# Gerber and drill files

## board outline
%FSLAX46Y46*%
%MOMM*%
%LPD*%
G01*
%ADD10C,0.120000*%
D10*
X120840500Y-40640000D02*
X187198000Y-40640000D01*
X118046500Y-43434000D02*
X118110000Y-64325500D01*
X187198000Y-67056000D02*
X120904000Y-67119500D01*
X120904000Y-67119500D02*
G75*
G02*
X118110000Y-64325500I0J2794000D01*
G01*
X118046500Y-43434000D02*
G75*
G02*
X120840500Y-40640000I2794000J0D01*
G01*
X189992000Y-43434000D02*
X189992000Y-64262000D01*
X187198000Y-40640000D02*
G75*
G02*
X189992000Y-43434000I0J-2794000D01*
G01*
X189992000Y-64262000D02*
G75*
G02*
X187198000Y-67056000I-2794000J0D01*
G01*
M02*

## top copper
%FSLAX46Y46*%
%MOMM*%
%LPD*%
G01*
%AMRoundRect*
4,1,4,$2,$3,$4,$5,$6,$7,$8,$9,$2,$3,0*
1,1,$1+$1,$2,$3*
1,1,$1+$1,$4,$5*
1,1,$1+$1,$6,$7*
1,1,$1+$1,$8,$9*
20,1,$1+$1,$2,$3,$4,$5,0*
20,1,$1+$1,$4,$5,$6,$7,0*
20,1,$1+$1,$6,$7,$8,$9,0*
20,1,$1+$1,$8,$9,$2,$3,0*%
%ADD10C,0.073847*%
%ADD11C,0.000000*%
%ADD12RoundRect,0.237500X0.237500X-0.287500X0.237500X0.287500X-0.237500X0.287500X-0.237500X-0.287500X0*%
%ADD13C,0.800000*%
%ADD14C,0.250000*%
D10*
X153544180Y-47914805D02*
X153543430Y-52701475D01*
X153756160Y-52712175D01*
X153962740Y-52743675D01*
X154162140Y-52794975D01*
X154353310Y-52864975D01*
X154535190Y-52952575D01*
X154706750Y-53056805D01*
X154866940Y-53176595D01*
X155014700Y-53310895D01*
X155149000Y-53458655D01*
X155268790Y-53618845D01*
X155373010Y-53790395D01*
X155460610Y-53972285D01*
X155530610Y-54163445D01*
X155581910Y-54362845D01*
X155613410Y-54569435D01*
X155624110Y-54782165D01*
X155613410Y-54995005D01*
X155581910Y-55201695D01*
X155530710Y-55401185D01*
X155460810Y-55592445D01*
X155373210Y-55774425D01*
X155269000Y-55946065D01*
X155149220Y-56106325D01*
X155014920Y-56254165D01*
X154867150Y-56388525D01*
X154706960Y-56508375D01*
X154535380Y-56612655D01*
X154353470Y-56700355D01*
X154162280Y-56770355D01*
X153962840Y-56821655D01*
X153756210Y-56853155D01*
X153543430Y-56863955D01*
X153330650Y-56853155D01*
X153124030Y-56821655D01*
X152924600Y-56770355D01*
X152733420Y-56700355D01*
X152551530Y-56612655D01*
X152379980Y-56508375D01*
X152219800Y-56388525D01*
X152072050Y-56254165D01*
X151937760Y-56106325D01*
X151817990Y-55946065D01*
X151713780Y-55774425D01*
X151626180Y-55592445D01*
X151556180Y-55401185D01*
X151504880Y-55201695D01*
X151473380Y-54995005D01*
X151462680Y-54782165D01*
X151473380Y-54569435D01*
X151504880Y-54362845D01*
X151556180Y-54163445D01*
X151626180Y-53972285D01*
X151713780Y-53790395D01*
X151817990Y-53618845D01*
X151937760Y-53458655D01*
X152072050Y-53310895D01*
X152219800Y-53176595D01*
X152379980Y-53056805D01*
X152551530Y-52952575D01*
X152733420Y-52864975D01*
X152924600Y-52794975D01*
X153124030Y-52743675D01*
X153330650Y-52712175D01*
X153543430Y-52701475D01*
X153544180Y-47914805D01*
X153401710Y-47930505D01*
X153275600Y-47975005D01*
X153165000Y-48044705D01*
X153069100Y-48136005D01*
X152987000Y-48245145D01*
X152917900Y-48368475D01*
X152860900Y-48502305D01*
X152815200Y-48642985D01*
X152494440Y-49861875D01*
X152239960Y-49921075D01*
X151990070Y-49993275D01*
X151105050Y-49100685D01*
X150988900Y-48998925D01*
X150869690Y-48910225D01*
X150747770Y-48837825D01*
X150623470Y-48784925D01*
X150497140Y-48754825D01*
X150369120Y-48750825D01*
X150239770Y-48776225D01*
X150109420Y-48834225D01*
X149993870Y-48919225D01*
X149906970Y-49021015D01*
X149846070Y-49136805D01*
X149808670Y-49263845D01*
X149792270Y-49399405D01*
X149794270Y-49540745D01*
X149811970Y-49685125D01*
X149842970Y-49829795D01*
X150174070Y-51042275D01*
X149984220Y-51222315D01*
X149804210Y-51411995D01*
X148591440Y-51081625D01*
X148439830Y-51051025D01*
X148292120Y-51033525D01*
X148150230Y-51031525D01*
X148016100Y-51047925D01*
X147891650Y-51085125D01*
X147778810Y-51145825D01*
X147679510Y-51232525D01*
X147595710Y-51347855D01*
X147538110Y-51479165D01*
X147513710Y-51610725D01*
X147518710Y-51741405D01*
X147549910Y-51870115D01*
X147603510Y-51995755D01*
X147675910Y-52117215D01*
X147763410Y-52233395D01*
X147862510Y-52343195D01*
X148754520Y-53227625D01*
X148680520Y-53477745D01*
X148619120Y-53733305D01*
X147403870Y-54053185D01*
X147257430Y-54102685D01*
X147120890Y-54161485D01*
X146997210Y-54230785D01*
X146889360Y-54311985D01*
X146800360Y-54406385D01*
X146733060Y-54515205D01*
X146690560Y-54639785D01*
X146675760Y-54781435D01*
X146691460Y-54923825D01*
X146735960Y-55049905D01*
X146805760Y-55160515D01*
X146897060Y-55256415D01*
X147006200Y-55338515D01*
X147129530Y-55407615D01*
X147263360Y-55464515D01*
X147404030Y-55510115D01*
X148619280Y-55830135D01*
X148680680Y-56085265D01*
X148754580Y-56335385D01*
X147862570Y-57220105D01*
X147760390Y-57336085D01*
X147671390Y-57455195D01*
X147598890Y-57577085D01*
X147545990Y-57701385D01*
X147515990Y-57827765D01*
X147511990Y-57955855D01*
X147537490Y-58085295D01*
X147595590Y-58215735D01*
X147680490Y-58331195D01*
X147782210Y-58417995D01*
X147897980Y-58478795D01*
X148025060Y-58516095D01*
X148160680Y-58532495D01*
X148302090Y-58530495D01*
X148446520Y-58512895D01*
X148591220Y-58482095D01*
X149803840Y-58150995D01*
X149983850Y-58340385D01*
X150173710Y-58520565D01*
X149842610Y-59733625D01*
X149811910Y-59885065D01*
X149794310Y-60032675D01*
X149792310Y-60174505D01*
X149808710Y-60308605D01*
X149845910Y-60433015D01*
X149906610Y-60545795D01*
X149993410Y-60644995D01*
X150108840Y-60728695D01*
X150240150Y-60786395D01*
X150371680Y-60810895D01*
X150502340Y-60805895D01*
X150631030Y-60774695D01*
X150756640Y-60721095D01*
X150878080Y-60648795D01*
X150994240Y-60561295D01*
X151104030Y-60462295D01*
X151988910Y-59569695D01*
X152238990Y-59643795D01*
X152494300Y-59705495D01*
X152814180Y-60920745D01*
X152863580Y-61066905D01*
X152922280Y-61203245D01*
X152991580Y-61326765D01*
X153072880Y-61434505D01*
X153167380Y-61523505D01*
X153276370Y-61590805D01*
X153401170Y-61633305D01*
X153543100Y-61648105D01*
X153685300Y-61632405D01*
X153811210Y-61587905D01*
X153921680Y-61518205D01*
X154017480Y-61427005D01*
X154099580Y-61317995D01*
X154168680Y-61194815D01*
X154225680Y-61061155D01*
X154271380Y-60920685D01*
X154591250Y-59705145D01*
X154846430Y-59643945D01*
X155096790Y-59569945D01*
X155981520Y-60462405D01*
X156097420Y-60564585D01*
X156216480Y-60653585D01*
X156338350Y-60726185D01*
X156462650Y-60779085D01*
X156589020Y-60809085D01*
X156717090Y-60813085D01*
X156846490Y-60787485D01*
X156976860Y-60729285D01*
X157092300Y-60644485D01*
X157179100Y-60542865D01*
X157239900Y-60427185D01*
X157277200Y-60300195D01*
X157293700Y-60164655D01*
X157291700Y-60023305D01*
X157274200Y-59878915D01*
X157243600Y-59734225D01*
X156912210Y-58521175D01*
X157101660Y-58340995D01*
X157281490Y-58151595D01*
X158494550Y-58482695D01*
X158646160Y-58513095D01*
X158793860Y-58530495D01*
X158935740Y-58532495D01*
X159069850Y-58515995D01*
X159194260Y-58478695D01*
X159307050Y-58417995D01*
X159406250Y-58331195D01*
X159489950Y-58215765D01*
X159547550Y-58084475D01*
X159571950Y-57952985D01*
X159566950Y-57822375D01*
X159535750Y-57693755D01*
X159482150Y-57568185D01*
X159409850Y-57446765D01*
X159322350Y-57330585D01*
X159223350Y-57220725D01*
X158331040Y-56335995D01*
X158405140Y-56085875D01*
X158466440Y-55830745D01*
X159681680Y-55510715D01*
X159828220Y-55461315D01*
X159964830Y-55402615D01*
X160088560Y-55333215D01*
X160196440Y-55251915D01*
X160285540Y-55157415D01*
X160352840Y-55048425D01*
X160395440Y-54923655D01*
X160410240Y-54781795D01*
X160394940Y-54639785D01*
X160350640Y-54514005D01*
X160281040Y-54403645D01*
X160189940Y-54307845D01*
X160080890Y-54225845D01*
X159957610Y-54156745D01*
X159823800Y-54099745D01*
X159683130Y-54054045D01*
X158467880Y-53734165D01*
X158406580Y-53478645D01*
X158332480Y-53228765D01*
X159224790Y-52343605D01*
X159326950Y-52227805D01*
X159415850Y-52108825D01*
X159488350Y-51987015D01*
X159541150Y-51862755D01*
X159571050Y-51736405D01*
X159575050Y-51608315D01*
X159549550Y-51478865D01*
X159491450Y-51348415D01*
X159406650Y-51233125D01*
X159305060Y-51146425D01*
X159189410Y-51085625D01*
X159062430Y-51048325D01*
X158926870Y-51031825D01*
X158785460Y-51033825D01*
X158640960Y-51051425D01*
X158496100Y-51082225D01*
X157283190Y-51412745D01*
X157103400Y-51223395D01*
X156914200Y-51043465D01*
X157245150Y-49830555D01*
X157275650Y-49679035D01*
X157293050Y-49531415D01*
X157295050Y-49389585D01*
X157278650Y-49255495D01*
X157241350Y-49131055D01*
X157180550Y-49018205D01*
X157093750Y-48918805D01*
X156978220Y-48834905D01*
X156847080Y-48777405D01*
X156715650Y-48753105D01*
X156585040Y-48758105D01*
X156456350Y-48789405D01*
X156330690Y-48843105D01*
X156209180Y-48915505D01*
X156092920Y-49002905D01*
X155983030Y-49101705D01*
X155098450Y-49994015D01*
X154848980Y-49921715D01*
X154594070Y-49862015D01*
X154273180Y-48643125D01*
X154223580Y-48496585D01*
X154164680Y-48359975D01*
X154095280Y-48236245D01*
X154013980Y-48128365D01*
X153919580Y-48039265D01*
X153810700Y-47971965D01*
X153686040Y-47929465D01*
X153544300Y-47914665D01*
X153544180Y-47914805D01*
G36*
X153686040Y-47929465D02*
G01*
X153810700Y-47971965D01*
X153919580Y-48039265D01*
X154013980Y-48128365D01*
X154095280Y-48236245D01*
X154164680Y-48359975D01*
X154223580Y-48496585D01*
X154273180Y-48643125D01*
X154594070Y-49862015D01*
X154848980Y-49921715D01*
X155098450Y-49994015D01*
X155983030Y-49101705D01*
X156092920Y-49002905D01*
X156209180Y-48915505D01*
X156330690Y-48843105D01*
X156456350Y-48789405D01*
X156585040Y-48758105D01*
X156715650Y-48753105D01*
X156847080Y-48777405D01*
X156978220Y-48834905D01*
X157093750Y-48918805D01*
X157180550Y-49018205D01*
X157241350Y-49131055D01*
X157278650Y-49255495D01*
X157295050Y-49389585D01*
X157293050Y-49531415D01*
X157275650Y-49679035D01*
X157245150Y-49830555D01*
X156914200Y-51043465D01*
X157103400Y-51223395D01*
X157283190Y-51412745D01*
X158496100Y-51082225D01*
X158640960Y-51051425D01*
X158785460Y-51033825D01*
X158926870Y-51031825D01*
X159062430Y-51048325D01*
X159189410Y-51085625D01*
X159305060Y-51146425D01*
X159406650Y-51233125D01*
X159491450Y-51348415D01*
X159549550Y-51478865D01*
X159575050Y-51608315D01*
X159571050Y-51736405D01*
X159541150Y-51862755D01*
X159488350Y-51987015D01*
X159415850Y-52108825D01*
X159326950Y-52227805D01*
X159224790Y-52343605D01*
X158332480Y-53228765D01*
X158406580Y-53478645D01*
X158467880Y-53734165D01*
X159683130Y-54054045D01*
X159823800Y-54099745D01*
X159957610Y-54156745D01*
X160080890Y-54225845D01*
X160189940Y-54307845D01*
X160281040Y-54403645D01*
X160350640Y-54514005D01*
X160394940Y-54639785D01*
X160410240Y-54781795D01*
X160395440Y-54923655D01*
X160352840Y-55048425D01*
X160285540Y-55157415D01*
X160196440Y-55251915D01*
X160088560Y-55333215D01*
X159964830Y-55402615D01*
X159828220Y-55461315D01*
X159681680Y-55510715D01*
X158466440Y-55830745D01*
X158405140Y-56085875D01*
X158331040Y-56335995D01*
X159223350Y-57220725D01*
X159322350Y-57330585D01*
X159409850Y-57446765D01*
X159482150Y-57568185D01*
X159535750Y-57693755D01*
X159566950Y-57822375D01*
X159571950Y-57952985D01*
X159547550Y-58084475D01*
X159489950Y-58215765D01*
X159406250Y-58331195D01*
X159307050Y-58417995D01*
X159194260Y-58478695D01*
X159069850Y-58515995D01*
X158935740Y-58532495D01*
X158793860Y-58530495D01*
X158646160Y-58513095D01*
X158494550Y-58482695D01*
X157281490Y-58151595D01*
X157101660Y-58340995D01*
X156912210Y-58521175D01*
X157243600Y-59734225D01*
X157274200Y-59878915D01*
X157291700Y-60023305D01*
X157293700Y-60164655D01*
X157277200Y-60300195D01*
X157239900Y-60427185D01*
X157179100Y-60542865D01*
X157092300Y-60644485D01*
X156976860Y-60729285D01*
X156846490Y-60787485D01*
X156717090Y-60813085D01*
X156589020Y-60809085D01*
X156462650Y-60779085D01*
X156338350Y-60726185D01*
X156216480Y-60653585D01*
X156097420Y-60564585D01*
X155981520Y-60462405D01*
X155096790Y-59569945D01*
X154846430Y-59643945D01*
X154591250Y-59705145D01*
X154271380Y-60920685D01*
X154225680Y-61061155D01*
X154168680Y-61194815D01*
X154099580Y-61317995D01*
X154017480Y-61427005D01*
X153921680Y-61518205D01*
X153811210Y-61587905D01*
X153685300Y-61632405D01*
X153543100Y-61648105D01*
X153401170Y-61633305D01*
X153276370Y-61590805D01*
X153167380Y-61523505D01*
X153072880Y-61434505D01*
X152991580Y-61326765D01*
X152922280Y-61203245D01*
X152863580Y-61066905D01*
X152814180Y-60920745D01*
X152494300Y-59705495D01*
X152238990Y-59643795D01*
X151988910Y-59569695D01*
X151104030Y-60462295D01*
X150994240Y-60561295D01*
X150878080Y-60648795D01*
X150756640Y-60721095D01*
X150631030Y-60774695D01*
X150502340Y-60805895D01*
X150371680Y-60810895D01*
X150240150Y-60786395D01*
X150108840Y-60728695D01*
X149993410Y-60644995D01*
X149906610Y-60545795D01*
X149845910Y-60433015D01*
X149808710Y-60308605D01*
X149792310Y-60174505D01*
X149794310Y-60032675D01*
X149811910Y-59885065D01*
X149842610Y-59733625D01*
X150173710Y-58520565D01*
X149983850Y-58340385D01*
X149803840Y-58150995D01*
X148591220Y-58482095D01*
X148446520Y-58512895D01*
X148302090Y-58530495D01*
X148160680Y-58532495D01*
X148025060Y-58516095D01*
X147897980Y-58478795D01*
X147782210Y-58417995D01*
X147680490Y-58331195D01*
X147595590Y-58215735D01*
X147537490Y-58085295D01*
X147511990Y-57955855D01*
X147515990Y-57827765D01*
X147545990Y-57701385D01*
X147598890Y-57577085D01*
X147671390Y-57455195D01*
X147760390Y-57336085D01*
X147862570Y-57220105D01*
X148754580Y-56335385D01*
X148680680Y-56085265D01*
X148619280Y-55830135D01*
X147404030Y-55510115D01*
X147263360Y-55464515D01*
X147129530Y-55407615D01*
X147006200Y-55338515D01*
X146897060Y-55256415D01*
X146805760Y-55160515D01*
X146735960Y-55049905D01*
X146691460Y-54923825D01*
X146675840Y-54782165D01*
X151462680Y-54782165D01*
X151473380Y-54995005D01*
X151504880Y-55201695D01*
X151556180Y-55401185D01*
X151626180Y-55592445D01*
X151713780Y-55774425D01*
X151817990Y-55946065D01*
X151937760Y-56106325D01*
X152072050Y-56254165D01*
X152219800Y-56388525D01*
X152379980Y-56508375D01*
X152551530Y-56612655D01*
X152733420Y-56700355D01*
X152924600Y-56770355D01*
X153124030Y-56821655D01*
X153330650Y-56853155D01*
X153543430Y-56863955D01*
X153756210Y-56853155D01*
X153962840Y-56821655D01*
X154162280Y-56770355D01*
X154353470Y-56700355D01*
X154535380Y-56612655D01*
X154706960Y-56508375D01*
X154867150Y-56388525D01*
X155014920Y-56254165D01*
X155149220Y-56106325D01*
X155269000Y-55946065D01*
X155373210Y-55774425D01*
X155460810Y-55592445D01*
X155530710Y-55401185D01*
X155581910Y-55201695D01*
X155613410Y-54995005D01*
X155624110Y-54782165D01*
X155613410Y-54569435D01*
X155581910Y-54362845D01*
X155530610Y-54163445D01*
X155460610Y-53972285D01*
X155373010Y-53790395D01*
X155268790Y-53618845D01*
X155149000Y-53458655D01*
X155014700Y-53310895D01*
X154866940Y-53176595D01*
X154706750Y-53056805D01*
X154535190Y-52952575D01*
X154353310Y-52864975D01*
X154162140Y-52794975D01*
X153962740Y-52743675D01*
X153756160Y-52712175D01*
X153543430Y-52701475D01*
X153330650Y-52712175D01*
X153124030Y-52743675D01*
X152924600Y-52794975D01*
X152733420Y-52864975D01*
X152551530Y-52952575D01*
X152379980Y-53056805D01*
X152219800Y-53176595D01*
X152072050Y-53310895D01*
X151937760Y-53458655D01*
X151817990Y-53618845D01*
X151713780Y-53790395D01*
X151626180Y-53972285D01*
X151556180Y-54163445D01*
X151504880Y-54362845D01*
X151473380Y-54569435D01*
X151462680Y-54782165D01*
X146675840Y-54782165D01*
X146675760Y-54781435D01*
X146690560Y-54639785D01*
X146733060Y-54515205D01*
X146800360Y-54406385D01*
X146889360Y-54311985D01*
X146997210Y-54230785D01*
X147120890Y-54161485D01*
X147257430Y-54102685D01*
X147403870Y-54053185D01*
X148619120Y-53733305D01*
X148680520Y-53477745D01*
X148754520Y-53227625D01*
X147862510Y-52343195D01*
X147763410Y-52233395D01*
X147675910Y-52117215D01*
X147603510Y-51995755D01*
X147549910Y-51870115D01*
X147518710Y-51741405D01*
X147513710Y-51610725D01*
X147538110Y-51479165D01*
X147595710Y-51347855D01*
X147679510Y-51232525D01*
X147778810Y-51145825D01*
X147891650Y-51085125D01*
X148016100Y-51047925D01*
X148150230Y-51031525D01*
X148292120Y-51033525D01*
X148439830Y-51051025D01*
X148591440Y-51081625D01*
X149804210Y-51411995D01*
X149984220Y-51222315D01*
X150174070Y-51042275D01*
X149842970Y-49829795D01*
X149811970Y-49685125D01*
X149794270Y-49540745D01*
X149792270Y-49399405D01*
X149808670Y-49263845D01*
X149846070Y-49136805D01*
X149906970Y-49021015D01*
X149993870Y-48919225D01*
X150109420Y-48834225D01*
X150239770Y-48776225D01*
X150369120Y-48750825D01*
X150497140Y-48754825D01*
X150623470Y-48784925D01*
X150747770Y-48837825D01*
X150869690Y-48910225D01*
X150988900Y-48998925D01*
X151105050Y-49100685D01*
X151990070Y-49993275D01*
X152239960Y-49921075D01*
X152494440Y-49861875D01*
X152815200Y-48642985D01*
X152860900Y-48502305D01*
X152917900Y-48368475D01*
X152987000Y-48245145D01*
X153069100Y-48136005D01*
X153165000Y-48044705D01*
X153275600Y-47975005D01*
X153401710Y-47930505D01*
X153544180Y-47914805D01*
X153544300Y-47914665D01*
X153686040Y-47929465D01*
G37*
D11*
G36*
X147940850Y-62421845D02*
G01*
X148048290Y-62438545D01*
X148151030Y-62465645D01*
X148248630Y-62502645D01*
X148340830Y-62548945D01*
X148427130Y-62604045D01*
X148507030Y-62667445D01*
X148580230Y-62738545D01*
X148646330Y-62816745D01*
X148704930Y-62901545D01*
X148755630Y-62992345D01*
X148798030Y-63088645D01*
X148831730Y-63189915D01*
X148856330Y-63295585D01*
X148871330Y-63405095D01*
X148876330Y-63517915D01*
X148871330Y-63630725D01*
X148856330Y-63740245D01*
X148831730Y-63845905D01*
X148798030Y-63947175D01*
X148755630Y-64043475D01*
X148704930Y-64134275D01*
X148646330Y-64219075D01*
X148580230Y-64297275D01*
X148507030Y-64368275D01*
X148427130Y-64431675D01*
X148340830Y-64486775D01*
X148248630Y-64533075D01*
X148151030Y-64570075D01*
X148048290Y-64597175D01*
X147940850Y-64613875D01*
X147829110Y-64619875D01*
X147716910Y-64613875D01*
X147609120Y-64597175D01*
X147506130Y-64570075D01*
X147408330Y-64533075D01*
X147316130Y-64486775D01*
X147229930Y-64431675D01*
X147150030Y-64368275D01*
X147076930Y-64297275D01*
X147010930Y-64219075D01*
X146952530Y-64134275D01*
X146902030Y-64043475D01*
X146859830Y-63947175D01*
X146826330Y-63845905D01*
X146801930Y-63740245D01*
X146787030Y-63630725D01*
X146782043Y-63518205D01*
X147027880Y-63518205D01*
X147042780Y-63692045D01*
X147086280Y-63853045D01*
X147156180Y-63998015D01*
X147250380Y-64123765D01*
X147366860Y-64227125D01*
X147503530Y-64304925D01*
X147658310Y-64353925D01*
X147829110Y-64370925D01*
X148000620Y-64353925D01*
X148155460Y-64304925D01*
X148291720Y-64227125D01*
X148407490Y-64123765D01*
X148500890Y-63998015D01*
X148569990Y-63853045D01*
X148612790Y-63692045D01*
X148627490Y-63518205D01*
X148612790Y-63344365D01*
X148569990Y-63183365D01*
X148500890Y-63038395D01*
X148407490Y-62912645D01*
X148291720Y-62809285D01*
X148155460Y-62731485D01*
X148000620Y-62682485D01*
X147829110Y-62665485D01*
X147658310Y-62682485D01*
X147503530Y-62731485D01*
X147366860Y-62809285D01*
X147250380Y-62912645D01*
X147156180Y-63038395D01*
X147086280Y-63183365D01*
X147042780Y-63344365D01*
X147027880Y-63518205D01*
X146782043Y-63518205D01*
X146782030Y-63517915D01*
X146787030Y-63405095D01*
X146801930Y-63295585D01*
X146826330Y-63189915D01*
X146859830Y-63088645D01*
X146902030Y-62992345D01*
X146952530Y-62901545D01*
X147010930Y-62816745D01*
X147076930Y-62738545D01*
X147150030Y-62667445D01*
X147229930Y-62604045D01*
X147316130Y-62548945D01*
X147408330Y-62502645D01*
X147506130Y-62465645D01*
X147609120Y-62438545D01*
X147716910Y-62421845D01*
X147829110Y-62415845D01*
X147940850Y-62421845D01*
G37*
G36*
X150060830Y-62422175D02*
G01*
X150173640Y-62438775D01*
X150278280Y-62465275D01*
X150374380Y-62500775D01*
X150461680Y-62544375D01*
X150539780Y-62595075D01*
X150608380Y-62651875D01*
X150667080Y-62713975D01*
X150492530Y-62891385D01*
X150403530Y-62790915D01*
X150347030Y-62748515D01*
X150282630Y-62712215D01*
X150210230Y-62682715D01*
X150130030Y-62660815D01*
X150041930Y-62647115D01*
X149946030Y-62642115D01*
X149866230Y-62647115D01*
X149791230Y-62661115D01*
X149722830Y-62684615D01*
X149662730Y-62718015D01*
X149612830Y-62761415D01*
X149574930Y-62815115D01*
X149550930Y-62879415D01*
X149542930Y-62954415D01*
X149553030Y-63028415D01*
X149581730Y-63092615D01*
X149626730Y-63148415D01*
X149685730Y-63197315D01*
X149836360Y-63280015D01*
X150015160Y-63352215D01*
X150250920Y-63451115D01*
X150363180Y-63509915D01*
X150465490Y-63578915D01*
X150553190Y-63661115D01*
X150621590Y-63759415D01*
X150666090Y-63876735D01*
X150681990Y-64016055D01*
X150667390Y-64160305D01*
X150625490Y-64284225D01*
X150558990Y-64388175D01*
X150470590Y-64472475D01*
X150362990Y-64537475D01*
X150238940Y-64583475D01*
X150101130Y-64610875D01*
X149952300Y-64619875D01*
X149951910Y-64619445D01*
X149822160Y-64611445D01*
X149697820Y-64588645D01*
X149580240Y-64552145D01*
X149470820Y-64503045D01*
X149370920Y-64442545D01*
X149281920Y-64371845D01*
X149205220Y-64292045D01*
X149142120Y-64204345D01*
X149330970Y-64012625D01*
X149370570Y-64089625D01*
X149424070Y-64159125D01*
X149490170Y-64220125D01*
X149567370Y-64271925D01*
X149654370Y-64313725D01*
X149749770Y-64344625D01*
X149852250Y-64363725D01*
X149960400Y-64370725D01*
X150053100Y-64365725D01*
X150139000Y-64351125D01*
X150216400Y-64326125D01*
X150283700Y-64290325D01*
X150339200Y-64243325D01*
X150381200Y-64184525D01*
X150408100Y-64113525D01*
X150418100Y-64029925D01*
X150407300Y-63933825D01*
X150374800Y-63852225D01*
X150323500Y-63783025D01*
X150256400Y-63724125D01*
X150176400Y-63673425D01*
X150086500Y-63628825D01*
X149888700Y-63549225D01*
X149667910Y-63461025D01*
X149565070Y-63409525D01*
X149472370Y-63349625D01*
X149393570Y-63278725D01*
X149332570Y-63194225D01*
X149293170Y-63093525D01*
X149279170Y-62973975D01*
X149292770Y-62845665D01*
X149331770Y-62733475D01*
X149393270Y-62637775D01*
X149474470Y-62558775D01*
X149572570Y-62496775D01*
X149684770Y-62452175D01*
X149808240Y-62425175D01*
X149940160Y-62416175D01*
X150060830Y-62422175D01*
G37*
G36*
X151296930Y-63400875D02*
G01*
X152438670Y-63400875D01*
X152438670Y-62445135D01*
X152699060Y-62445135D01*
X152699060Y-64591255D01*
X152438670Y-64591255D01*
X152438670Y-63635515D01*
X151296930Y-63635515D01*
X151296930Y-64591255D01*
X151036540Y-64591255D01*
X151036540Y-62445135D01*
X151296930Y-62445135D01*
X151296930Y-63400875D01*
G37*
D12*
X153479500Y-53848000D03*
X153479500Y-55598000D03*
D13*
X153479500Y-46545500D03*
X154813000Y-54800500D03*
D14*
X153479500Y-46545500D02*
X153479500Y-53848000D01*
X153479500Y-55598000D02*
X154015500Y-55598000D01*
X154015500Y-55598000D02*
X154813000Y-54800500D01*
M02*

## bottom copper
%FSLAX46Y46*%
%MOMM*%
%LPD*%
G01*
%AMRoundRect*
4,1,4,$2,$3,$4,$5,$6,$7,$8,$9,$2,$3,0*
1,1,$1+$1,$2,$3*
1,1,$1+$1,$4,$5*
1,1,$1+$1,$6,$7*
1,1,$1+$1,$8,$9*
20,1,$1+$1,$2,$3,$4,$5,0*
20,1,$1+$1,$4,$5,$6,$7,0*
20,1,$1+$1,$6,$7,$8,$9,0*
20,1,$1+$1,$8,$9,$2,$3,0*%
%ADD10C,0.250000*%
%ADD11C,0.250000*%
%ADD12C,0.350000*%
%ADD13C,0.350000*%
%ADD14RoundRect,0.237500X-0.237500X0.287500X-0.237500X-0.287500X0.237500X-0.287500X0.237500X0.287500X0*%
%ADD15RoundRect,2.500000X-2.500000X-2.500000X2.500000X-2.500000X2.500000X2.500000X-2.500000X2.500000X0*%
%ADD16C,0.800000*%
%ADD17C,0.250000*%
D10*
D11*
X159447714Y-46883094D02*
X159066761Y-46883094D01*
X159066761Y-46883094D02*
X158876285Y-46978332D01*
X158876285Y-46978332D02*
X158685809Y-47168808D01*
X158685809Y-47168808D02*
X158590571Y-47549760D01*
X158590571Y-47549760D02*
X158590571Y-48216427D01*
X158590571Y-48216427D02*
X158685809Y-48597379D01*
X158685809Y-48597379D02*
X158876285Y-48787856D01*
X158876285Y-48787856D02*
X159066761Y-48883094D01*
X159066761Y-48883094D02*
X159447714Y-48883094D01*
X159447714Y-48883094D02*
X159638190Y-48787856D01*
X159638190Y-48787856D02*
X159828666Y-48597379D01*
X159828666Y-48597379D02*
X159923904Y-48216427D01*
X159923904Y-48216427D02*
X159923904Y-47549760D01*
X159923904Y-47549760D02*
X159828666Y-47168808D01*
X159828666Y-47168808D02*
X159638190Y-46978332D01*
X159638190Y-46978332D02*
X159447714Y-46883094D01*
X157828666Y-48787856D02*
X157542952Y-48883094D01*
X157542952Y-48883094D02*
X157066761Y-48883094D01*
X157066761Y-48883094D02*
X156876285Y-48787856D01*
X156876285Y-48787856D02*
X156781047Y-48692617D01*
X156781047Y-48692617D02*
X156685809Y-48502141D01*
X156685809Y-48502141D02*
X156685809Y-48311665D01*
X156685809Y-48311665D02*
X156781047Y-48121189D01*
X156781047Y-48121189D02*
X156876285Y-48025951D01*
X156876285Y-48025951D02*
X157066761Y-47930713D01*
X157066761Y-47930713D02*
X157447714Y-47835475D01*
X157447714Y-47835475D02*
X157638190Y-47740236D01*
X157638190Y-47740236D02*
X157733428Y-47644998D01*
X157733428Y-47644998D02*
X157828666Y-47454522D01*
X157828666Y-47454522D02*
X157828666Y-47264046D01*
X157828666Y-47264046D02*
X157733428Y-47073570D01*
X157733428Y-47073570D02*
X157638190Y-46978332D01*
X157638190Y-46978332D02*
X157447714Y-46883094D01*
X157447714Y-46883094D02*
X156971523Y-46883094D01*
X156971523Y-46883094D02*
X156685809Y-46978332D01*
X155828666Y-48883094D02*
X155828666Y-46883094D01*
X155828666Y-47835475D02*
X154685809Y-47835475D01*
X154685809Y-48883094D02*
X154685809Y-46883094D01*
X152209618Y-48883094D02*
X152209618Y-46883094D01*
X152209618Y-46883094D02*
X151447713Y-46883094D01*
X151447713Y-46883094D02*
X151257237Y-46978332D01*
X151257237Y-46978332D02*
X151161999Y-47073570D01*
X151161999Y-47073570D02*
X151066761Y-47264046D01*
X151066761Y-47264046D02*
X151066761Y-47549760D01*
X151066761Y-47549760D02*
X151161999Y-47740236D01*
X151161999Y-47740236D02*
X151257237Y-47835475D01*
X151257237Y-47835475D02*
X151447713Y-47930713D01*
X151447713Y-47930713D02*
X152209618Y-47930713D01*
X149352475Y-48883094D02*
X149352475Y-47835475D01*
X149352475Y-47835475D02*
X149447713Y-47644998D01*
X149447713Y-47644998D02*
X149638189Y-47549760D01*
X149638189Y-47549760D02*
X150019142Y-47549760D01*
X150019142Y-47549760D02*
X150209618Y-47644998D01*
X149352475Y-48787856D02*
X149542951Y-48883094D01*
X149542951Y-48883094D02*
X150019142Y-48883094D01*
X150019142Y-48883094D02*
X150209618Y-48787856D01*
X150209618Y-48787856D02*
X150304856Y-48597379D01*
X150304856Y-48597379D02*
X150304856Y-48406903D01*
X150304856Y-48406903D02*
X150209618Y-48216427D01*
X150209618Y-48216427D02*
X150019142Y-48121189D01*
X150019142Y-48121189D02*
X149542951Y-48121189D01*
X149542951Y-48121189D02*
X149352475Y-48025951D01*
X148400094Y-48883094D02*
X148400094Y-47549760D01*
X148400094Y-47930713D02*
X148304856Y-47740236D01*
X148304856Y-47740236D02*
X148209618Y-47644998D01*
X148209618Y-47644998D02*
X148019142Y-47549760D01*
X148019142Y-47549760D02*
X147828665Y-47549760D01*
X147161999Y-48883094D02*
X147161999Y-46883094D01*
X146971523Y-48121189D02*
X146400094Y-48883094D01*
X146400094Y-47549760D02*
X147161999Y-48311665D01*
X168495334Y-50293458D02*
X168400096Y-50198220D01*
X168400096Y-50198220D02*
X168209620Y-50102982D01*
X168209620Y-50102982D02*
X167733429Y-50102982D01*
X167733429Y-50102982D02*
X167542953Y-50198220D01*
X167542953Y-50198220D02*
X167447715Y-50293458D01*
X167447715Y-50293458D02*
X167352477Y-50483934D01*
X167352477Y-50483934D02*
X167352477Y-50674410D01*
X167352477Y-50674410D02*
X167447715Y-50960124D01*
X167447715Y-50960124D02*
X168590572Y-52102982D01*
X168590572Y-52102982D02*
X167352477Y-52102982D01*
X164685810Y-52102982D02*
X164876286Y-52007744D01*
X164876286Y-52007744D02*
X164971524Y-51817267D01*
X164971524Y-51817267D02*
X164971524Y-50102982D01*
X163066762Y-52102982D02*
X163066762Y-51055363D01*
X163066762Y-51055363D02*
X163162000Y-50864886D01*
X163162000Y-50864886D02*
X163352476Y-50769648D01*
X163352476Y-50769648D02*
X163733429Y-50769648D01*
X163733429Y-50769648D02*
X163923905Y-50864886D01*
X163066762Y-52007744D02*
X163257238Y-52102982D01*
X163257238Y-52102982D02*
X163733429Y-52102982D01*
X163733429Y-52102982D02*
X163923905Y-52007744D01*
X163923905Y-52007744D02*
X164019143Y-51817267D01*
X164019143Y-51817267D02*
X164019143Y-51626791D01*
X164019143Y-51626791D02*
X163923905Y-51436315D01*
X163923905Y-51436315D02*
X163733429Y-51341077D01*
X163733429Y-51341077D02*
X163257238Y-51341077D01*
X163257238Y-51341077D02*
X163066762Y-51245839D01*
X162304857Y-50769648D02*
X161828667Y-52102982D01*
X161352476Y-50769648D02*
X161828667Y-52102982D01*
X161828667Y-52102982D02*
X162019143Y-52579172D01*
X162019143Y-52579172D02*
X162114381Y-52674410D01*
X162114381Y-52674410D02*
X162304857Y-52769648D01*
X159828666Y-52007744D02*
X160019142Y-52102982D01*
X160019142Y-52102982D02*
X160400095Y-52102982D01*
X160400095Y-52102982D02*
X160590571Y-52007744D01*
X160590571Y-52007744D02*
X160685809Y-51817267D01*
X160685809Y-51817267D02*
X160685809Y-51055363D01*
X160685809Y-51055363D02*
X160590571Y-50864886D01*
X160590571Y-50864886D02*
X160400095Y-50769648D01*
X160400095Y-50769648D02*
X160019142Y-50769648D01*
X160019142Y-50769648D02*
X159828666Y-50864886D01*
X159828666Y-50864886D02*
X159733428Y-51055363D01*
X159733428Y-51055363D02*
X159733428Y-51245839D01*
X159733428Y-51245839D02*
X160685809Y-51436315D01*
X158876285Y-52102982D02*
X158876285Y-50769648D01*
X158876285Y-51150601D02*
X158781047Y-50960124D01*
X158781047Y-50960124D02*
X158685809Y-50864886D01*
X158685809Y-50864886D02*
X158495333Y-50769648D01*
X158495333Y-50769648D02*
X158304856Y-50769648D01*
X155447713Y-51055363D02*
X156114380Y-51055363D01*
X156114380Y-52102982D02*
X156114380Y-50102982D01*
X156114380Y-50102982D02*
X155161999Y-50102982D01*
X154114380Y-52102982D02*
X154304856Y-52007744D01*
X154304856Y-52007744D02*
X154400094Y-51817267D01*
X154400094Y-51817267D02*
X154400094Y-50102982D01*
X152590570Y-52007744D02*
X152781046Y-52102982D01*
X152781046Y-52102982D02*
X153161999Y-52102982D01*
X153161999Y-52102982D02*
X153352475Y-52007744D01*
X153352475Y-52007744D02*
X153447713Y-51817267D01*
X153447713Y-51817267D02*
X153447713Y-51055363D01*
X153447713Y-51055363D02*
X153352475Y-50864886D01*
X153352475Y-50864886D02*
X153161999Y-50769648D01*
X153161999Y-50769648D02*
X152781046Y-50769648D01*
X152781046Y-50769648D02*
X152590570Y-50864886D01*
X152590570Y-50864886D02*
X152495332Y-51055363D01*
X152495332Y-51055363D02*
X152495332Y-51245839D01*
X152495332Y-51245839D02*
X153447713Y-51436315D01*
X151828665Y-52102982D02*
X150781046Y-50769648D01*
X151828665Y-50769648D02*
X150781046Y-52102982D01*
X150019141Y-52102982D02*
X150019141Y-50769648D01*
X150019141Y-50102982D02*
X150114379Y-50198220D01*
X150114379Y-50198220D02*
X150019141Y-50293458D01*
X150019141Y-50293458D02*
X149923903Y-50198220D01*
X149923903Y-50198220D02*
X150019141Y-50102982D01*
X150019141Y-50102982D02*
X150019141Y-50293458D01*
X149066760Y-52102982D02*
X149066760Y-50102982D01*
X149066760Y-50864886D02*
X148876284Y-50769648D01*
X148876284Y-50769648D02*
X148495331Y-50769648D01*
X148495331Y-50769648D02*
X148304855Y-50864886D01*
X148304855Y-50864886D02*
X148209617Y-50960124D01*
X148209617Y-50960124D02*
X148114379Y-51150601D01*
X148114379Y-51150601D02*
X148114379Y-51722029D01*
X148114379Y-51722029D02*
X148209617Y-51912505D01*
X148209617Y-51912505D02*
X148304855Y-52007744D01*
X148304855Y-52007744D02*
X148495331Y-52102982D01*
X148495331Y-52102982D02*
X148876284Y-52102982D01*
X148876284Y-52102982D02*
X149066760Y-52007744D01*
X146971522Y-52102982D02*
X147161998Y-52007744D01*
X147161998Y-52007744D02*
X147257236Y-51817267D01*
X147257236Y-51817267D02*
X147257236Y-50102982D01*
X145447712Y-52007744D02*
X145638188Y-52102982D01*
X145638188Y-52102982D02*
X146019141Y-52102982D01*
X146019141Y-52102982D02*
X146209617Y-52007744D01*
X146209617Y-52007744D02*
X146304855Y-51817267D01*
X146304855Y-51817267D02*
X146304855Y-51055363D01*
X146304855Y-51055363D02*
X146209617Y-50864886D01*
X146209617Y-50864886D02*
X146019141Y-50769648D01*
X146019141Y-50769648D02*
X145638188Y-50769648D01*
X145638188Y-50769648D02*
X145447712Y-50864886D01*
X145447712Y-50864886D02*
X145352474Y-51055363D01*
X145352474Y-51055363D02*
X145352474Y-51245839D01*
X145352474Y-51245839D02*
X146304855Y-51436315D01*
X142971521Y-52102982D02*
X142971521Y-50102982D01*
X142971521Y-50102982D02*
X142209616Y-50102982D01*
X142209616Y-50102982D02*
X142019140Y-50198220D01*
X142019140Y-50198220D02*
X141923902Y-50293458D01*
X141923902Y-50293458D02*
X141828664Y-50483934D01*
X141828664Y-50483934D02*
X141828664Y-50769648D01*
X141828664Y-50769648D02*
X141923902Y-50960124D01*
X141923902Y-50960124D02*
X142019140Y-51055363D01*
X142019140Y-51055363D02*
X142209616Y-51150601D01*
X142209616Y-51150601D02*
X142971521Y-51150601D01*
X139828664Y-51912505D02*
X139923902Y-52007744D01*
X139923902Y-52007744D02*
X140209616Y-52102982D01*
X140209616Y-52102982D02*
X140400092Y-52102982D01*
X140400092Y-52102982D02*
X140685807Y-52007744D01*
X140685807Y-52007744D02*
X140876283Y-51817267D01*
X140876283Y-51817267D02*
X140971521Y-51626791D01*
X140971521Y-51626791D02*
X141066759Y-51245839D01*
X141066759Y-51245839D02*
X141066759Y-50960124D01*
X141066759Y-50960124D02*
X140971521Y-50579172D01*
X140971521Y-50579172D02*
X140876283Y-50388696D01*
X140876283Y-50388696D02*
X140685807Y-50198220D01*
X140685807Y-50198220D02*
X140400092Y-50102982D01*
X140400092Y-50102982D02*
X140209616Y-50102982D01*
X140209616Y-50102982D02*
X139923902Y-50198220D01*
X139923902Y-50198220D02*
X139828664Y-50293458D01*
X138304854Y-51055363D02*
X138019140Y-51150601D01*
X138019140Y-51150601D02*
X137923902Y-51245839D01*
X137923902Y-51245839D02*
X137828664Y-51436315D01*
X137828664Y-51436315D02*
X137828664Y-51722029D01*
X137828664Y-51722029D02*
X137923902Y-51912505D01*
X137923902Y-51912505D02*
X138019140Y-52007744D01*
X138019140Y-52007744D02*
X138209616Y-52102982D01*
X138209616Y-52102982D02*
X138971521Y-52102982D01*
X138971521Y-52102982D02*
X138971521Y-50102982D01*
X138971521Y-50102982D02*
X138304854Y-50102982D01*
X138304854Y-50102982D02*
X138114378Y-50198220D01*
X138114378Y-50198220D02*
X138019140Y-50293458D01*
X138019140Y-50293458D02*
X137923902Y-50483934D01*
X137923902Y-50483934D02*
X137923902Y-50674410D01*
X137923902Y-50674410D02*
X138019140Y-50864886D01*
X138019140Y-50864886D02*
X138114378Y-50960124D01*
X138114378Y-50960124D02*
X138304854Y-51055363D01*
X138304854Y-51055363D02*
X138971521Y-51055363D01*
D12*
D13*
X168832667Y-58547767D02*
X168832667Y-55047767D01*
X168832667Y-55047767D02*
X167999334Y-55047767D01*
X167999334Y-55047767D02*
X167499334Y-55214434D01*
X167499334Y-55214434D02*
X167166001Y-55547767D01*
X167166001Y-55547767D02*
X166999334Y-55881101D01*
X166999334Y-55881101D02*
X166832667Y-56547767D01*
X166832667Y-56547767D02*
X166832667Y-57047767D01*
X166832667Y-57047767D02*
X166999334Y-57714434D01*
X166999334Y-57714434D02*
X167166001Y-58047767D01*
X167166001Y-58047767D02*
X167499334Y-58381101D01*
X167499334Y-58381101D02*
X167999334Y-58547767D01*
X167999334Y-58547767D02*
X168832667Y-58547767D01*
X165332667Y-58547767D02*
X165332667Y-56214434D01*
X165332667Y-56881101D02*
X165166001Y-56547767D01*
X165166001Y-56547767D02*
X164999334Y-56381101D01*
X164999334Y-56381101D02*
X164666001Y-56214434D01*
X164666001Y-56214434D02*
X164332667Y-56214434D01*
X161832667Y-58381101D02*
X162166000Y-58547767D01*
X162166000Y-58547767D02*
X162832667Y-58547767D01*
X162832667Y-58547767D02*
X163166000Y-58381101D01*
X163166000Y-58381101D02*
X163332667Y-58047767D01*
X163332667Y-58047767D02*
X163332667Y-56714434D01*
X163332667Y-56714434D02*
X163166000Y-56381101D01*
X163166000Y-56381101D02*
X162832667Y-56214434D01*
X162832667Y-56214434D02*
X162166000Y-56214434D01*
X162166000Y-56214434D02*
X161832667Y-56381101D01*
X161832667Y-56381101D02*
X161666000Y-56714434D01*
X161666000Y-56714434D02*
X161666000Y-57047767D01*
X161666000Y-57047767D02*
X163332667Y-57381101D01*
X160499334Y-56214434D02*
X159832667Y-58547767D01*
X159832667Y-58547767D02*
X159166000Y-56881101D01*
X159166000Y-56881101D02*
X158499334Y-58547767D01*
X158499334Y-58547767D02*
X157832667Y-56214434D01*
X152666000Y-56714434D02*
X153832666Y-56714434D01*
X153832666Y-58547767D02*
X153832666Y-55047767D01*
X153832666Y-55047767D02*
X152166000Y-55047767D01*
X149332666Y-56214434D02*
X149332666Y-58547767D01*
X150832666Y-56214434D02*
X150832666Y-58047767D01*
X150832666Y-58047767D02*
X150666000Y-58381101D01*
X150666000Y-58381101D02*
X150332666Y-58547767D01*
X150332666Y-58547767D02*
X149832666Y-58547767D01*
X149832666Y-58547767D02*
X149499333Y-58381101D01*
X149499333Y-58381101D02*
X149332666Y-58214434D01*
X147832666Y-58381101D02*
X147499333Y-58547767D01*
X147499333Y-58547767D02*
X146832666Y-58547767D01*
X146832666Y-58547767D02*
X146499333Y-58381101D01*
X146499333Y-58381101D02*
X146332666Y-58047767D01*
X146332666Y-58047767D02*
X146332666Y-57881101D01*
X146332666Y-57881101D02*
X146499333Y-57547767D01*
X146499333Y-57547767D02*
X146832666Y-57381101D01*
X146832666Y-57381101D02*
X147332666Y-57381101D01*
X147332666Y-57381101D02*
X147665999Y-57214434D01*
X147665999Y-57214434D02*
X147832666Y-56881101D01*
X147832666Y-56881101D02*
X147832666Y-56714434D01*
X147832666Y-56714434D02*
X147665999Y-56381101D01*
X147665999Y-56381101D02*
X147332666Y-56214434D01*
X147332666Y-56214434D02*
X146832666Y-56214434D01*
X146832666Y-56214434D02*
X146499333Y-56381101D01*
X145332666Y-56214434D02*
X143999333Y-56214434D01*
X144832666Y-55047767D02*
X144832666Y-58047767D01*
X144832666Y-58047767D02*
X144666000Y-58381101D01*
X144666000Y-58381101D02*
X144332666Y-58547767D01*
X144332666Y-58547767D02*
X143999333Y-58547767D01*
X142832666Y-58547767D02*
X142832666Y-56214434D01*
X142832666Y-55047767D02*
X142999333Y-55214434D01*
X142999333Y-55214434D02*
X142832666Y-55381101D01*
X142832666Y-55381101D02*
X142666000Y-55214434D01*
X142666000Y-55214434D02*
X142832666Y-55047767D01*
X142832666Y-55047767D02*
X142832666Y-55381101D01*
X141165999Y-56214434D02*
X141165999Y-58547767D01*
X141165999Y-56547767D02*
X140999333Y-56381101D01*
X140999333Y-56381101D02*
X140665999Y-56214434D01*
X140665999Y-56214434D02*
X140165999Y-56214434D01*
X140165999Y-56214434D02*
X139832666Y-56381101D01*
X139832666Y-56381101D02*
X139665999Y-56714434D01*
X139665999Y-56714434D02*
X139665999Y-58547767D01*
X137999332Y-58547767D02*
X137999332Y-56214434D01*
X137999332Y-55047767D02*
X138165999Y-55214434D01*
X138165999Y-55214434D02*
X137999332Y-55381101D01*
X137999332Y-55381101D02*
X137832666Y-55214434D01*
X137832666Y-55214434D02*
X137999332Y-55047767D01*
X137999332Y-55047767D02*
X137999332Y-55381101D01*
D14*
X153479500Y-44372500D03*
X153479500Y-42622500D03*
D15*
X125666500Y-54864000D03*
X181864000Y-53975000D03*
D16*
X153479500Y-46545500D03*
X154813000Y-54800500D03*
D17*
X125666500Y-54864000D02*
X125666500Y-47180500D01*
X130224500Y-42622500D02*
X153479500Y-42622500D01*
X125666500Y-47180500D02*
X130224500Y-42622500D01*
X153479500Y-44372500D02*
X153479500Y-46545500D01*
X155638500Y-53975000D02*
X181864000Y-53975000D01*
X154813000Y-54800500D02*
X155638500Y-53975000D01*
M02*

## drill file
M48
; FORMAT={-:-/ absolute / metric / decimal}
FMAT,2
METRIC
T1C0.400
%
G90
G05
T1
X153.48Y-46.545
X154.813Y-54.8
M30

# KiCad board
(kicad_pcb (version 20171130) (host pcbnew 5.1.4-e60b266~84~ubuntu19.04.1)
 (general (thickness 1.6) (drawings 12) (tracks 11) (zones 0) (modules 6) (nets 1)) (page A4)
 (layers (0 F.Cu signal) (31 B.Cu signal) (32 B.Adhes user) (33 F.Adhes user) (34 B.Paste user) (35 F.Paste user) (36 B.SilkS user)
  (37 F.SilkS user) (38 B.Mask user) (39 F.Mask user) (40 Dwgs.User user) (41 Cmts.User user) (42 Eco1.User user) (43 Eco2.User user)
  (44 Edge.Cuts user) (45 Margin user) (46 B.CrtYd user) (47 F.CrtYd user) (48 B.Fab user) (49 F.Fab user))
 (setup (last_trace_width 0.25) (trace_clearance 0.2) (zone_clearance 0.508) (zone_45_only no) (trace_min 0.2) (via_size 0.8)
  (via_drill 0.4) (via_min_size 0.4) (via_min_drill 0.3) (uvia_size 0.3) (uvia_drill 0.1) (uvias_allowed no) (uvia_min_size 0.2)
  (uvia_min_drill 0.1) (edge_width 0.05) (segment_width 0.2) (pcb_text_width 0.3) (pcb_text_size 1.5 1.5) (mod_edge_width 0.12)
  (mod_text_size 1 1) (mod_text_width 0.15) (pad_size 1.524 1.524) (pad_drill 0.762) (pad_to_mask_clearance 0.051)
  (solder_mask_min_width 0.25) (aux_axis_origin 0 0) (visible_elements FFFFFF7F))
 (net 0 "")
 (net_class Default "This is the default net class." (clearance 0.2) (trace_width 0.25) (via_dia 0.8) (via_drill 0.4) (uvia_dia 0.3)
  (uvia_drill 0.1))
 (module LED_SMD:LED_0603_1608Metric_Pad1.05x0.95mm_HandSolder (layer F.Cu) (at 153.4795 54.723 90)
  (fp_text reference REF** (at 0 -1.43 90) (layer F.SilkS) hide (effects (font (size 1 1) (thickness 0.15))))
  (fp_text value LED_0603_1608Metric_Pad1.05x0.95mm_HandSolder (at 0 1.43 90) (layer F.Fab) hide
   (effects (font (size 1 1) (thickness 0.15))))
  (pad 2 smd roundrect (at 0.875 0 90) (size 1.05 0.95) (layers F.Cu F.Paste F.Mask) (roundrect_rratio 0.25))
  (pad 1 smd roundrect (at -0.875 0 90) (size 1.05 0.95) (layers F.Cu F.Paste F.Mask) (roundrect_rratio 0.25)))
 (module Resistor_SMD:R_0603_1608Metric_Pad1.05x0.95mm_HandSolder (layer B.Cu) (at 153.4795 43.4975 270)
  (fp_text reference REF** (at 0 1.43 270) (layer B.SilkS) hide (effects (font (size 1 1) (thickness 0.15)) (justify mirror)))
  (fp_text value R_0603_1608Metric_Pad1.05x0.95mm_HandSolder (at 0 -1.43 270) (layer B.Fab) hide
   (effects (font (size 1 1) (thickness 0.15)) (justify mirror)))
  (pad 2 smd roundrect (at 0.875 0 270) (size 1.05 0.95) (layers B.Cu B.Paste B.Mask) (roundrect_rratio 0.25))
  (pad 1 smd roundrect (at -0.875 0 270) (size 1.05 0.95) (layers B.Cu B.Paste B.Mask) (roundrect_rratio 0.25)))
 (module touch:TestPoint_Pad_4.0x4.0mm (layer B.Cu) (at 125.6665 54.864)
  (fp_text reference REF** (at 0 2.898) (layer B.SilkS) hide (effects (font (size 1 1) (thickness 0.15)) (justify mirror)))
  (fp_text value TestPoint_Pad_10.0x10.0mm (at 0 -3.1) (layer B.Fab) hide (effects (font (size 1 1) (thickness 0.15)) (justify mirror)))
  (pad 1 smd roundrect (at 0 0) (size 10 10) (layers B.Cu B.Mask) (roundrect_rratio 0.25)))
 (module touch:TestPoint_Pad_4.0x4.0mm (layer B.Cu) (at 181.864 53.975)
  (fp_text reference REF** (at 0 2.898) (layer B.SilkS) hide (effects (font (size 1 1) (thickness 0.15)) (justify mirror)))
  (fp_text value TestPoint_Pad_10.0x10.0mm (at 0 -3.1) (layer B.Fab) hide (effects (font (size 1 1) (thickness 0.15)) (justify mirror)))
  (pad 1 smd roundrect (at 0 0) (size 10 10) (layers B.Cu B.Mask) (roundrect_rratio 0.25)))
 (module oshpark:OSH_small (layer F.Cu) (at 153.543 56.3245)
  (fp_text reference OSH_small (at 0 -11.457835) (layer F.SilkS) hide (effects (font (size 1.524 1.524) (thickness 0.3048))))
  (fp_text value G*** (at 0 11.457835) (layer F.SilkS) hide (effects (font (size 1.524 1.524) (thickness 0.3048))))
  (fp_poly
   (pts (xy 0.00118 -8.409695) (xy 0.00043 -3.623025) (xy 0.21316 -3.612325) (xy 0.41974 -3.580825) (xy 0.61914 -3.529525)
    (xy 0.81031 -3.459525) (xy 0.99219 -3.371925) (xy 1.16375 -3.267695) (xy 1.32394 -3.147905) (xy 1.4717 -3.013605) (xy 1.606 -2.865845)
    (xy 1.72579 -2.705655) (xy 1.83001 -2.534105) (xy 1.91761 -2.352215) (xy 1.98761 -2.161055) (xy 2.03891 -1.961655)
    (xy 2.07041 -1.755065) (xy 2.08111 -1.542335) (xy 2.07041 -1.329495) (xy 2.03891 -1.122805) (xy 1.98771 -0.923315)
    (xy 1.91781 -0.732055) (xy 1.83021 -0.550075) (xy 1.726 -0.378435) (xy 1.60622 -0.218175) (xy 1.47192 -0.070335) (xy 1.32415 0.064025)
    (xy 1.16396 0.183875) (xy 0.99238 0.288155) (xy 0.81047 0.375855) (xy 0.61928 0.445855) (xy 0.41984 0.497155) (xy 0.21321 0.528655)
    (xy 0.00043 0.539455) (xy -0.21235 0.528655) (xy -0.41897 0.497155) (xy -0.6184 0.445855) (xy -0.80958 0.375855) (xy -0.99147 0.288155)
    (xy -1.16302 0.183875) (xy -1.3232 0.064025) (xy -1.47095 -0.070335) (xy -1.60524 -0.218175) (xy -1.72501 -0.378435)
    (xy -1.82922 -0.550075) (xy -1.91682 -0.732055) (xy -1.98682 -0.923315) (xy -2.03812 -1.122805) (xy -2.06962 -1.329495)
    (xy -2.08032 -1.542335) (xy -2.06962 -1.755065) (xy -2.03812 -1.961655) (xy -1.98682 -2.161055) (xy -1.91682 -2.352215)
    (xy -1.82922 -2.534105) (xy -1.72501 -2.705655) (xy -1.60524 -2.865845) (xy -1.47095 -3.013605) (xy -1.3232 -3.147905)
    (xy -1.16302 -3.267695) (xy -0.99147 -3.371925) (xy -0.80958 -3.459525) (xy -0.6184 -3.529525) (xy -0.41897 -3.580825)
    (xy -0.21235 -3.612325) (xy 0.00043 -3.623025) (xy 0.00118 -8.409695) (xy -0.14129 -8.393995) (xy -0.2674 -8.349495)
    (xy -0.378 -8.279795) (xy -0.4739 -8.188495) (xy -0.556 -8.079355) (xy -0.6251 -7.956025) (xy -0.6821 -7.822195) (xy -0.7278 -7.681515)
    (xy -1.04856 -6.462625) (xy -1.30304 -6.403425) (xy -1.55293 -6.331225) (xy -2.43795 -7.223815) (xy -2.5541 -7.325575)
    (xy -2.67331 -7.414275) (xy -2.79523 -7.486675) (xy -2.91953 -7.539575) (xy -3.04586 -7.569675) (xy -3.17388 -7.573675)
    (xy -3.30323 -7.548275) (xy -3.43358 -7.490275) (xy -3.54913 -7.405275) (xy -3.63603 -7.303485) (xy -3.69693 -7.187695)
    (xy -3.73433 -7.060655) (xy -3.75073 -6.925095) (xy -3.74873 -6.783755) (xy -3.73103 -6.639375) (xy -3.70003 -6.494705)
    (xy -3.36893 -5.282225) (xy -3.55878 -5.102185) (xy -3.73879 -4.912505) (xy -4.95156 -5.242875) (xy -5.10317 -5.273475)
    (xy -5.25088 -5.290975) (xy -5.39277 -5.292975) (xy -5.5269 -5.276575) (xy -5.65135 -5.239375) (xy -5.76419 -5.178675)
    (xy -5.86349 -5.091975) (xy -5.94729 -4.976645) (xy -6.00489 -4.845335) (xy -6.02929 -4.713775) (xy -6.02429 -4.583095)
    (xy -5.99309 -4.454385) (xy -5.93949 -4.328745) (xy -5.86709 -4.207285) (xy -5.77959 -4.091105) (xy -5.68049 -3.981305)
    (xy -4.78848 -3.096875) (xy -4.86248 -2.846755) (xy -4.92388 -2.591195) (xy -6.13913 -2.271315) (xy -6.28557 -2.221815)
    (xy -6.42211 -2.163015) (xy -6.54579 -2.093715) (xy -6.65364 -2.012515) (xy -6.74264 -1.918115) (xy -6.80994 -1.809295)
    (xy -6.85244 -1.684715) (xy -6.86724 -1.543065) (xy -6.85154 -1.400675) (xy -6.80704 -1.274595) (xy -6.73724 -1.163985)
    (xy -6.64594 -1.068085) (xy -6.5368 -0.985985) (xy -6.41347 -0.916885) (xy -6.27964 -0.859985) (xy -6.13897 -0.814385)
    (xy -4.92372 -0.494365) (xy -4.86232 -0.239235) (xy -4.78842 0.010885) (xy -5.68043 0.895605) (xy -5.78261 1.011585)
    (xy -5.87161 1.130695) (xy -5.94411 1.252585) (xy -5.99701 1.376885) (xy -6.02701 1.503265) (xy -6.03101 1.631355)
    (xy -6.00551 1.760795) (xy -5.94741 1.891235) (xy -5.86251 2.006695) (xy -5.76079 2.093495) (xy -5.64502 2.154295)
    (xy -5.51794 2.191595) (xy -5.38232 2.207995) (xy -5.24091 2.205995) (xy -5.09648 2.188395) (xy -4.95178 2.157595)
    (xy -3.73916 1.826495) (xy -3.55915 2.015885) (xy -3.36929 2.196065) (xy -3.70039 3.409125) (xy -3.73109 3.560565)
    (xy -3.74869 3.708175) (xy -3.75069 3.850005) (xy -3.73429 3.984105) (xy -3.69709 4.108515) (xy -3.63639 4.221295)
    (xy -3.54959 4.320495) (xy -3.43416 4.404195) (xy -3.30285 4.461895) (xy -3.17132 4.486395) (xy -3.04066 4.481395)
    (xy -2.91197 4.450195) (xy -2.78636 4.396595) (xy -2.66492 4.324295) (xy -2.54876 4.236795) (xy -2.43897 4.137795)
    (xy -1.55409 3.245195) (xy -1.30401 3.319295) (xy -1.0487 3.380995) (xy -0.72882 4.596245) (xy -0.67942 4.742405) (xy -0.62072 4.878745)
    (xy -0.55142 5.002265) (xy -0.47012 5.110005) (xy -0.37562 5.199005) (xy -0.26663 5.266305) (xy -0.14183 5.308805) (xy 0.0001 5.323605)
    (xy 0.1423 5.307905) (xy 0.26821 5.263405) (xy 0.37868 5.193705) (xy 0.47448 5.102505) (xy 0.55658 4.993495) (xy 0.62568 4.870315)
    (xy 0.68268 4.736655) (xy 0.72838 4.596185) (xy 1.04825 3.380645) (xy 1.30343 3.319445) (xy 1.55379 3.245445) (xy 2.43852 4.137905)
    (xy 2.55442 4.240085) (xy 2.67348 4.329085) (xy 2.79535 4.401685) (xy 2.91965 4.454585) (xy 3.04602 4.484585) (xy 3.17409 4.488585)
    (xy 3.30349 4.462985) (xy 3.43386 4.404785) (xy 3.5493 4.319985) (xy 3.6361 4.218365) (xy 3.6969 4.102685) (xy 3.7342 3.975695)
    (xy 3.7507 3.840155) (xy 3.7487 3.698805) (xy 3.7312 3.554415) (xy 3.7006 3.409725) (xy 3.36921 2.196675) (xy 3.55866 2.016495)
    (xy 3.73849 1.827095) (xy 4.95155 2.158195) (xy 5.10316 2.188595) (xy 5.25086 2.205995) (xy 5.39274 2.207995) (xy 5.52685 2.191495)
    (xy 5.65126 2.154195) (xy 5.76405 2.093495) (xy 5.86325 2.006695) (xy 5.94695 1.891265) (xy 6.00455 1.759975) (xy 6.02895 1.628485)
    (xy 6.02395 1.497875) (xy 5.99275 1.369255) (xy 5.93915 1.243685) (xy 5.86685 1.122265) (xy 5.77935 1.006085) (xy 5.68035 0.896225)
    (xy 4.78804 0.011495) (xy 4.86214 -0.238625) (xy 4.92344 -0.493755) (xy 6.13868 -0.813785) (xy 6.28522 -0.863185) (xy 6.42183 -0.921885)
    (xy 6.54556 -0.991285) (xy 6.65344 -1.072585) (xy 6.74254 -1.167085) (xy 6.80984 -1.276075) (xy 6.85244 -1.400845)
    (xy 6.86724 -1.542705) (xy 6.85194 -1.684715) (xy 6.80764 -1.810495) (xy 6.73804 -1.920855) (xy 6.64694 -2.016655)
    (xy 6.53789 -2.098655) (xy 6.41461 -2.167755) (xy 6.2808 -2.224755) (xy 6.14013 -2.270455) (xy 4.92488 -2.590335) (xy 4.86358 -2.845855)
    (xy 4.78948 -3.095735) (xy 5.68179 -3.980895) (xy 5.78395 -4.096695) (xy 5.87285 -4.215675) (xy 5.94535 -4.337485)
    (xy 5.99815 -4.461745) (xy 6.02805 -4.588095) (xy 6.03205 -4.716185) (xy 6.00655 -4.845635) (xy 5.94845 -4.976085)
    (xy 5.86365 -5.091375) (xy 5.76206 -5.178075) (xy 5.64641 -5.238875) (xy 5.51943 -5.276175) (xy 5.38387 -5.292675)
    (xy 5.24246 -5.290675) (xy 5.09796 -5.273075) (xy 4.9531 -5.242275) (xy 3.74019 -4.911755) (xy 3.5604 -5.101105) (xy 3.3712 -5.281035)
    (xy 3.70215 -6.493945) (xy 3.73265 -6.645465) (xy 3.75005 -6.793085) (xy 3.75205 -6.934915) (xy 3.73565 -7.069005)
    (xy 3.69835 -7.193445) (xy 3.63755 -7.306295) (xy 3.55075 -7.405695) (xy 3.43522 -7.489595) (xy 3.30408 -7.547095)
    (xy 3.17265 -7.571395) (xy 3.04204 -7.566395) (xy 2.91335 -7.535095) (xy 2.78769 -7.481395) (xy 2.66618 -7.408995)
    (xy 2.54992 -7.321595) (xy 2.44003 -7.222795) (xy 1.55545 -6.330485) (xy 1.30598 -6.402785) (xy 1.05107 -6.462485)
    (xy 0.73018 -7.681375) (xy 0.68058 -7.827915) (xy 0.62168 -7.964525) (xy 0.55228 -8.088255) (xy 0.47098 -8.196135)
    (xy 0.37658 -8.285235) (xy 0.2677 -8.352535) (xy 0.14304 -8.395035) (xy 0.0013 -8.409835) (xy 0.00118 -8.409695))
   (layer F.Cu) (width 0.073847))
  (fp_poly
   (pts (xy -5.71389 8.295375) (xy -5.71389 8.046425) (xy -5.88469 8.029425) (xy -6.03947 7.980425) (xy -6.17614 7.902625)
    (xy -6.29262 7.799265) (xy -6.38682 7.673515) (xy -6.45672 7.528545) (xy -6.50022 7.367545) (xy -6.51512 7.193705)
    (xy -6.50022 7.019865) (xy -6.45672 6.858865) (xy -6.38682 6.713895) (xy -6.29262 6.588145) (xy -6.17614 6.484785)
    (xy -6.03947 6.406985) (xy -5.88469 6.357985) (xy -5.71389 6.340985) (xy -5.54238 6.357985) (xy -5.38754 6.406985)
    (xy -5.25128 6.484785) (xy -5.13551 6.588145) (xy -5.04211 6.713895) (xy -4.97301 6.858865) (xy -4.93021 7.019865)
    (xy -4.91551 7.193705) (xy -4.93021 7.367545) (xy -4.97301 7.528545) (xy -5.04211 7.673515) (xy -5.13551 7.799265)
    (xy -5.25128 7.902625) (xy -5.38754 7.980425) (xy -5.54238 8.029425) (xy -5.71389 8.046425) (xy -5.71389 8.295375)
    (xy -5.60215 8.289375) (xy -5.49471 8.272675) (xy -5.39197 8.245575) (xy -5.29437 8.208575) (xy -5.20217 8.162275)
    (xy -5.11587 8.107175) (xy -5.03597 8.043775) (xy -4.96277 7.972775) (xy -4.89667 7.894575) (xy -4.83807 7.809775)
    (xy -4.78737 7.718975) (xy -4.74497 7.622675) (xy -4.71127 7.521405) (xy -4.68667 7.415745) (xy -4.67167 7.306225)
    (xy -4.66667 7.193415) (xy -4.67167 7.080595) (xy -4.68667 6.971085) (xy -4.71127 6.865415) (xy -4.74497 6.764145)
    (xy -4.78737 6.667845) (xy -4.83807 6.577045) (xy -4.89667 6.492245) (xy -4.96277 6.414045) (xy -5.03597 6.342945)
    (xy -5.11587 6.279545) (xy -5.20217 6.224445) (xy -5.29437 6.178145) (xy -5.39197 6.141145) (xy -5.49471 6.114045)
    (xy -5.60215 6.097345) (xy -5.71389 6.091345) (xy -5.82609 6.097345) (xy -5.93388 6.114045) (xy -6.03687 6.141145)
    (xy -6.13467 6.178145) (xy -6.22687 6.224445) (xy -6.31307 6.279545) (xy -6.39297 6.342945) (xy -6.46607 6.414045)
    (xy -6.53207 6.492245) (xy -6.59047 6.577045) (xy -6.64097 6.667845) (xy -6.68317 6.764145) (xy -6.71667 6.865415)
    (xy -6.74107 6.971085) (xy -6.75597 7.080595) (xy -6.76097 7.193415) (xy -6.75597 7.306225) (xy -6.74107 7.415745)
    (xy -6.71667 7.521405) (xy -6.68317 7.622675) (xy -6.64097 7.718975) (xy -6.59047 7.809775) (xy -6.53207 7.894575)
    (xy -6.46607 7.972775) (xy -6.39297 8.043775) (xy -6.31307 8.107175) (xy -6.22687 8.162275) (xy -6.13467 8.208575)
    (xy -6.03687 8.245575) (xy -5.93388 8.272675) (xy -5.82609 8.289375) (xy -5.71389 8.295375))
   (layer F.Cu) (width 0))
  (fp_poly
   (pts (xy -3.5907 8.295375) (xy -3.44187 8.286375) (xy -3.30406 8.258975) (xy -3.18001 8.212975) (xy -3.07241 8.147975)
    (xy -2.98401 8.063675) (xy -2.91751 7.959725) (xy -2.87561 7.835805) (xy -2.86101 7.691555) (xy -2.87691 7.552235)
    (xy -2.92141 7.434915) (xy -2.98981 7.336615) (xy -3.07751 7.254415) (xy -3.17982 7.185415) (xy -3.29208 7.126615)
    (xy -3.52784 7.027715) (xy -3.70664 6.955515) (xy -3.85727 6.872815) (xy -3.91627 6.823915) (xy -3.96127 6.768115)
    (xy -3.98997 6.703915) (xy -4.00007 6.629915) (xy -3.99207 6.554915) (xy -3.96807 6.490615) (xy -3.93017 6.436915)
    (xy -3.88027 6.393515) (xy -3.82017 6.360115) (xy -3.75177 6.336615) (xy -3.67677 6.322615) (xy -3.59697 6.317615)
    (xy -3.50107 6.322615) (xy -3.41297 6.336315) (xy -3.33277 6.358215) (xy -3.26037 6.387715) (xy -3.19597 6.424015)
    (xy -3.13947 6.466415) (xy -3.05047 6.566885) (xy -2.87592 6.389475) (xy -2.93462 6.327375) (xy -3.00322 6.270575)
    (xy -3.08132 6.219875) (xy -3.16862 6.176275) (xy -3.26472 6.140775) (xy -3.36936 6.114275) (xy -3.48217 6.097675)
    (xy -3.60284 6.091675) (xy -3.73476 6.100675) (xy -3.85823 6.127675) (xy -3.97043 6.172275) (xy -4.06853 6.234275)
    (xy -4.14973 6.313275) (xy -4.21123 6.408975) (xy -4.25023 6.521165) (xy -4.26383 6.649475) (xy -4.24983 6.769025)
    (xy -4.21043 6.869725) (xy -4.14943 6.954225) (xy -4.07063 7.025125) (xy -3.97793 7.085025) (xy -3.87509 7.136525) (xy -3.6543 7.224725)
    (xy -3.4565 7.304325) (xy -3.3666 7.348925) (xy -3.2866 7.399625) (xy -3.2195 7.458525) (xy -3.1682 7.527725) (xy -3.1357 7.609325)
    (xy -3.1249 7.705425) (xy -3.1349 7.789025) (xy -3.1618 7.860025) (xy -3.2038 7.918825) (xy -3.2593 7.965825) (xy -3.3266 8.001625)
    (xy -3.404 8.026625) (xy -3.4899 8.041225) (xy -3.5826 8.046225) (xy -3.69075 8.039225) (xy -3.79323 8.020125) (xy -3.88863 7.989225)
    (xy -3.97563 7.947425) (xy -4.05283 7.895625) (xy -4.11893 7.834625) (xy -4.17243 7.765125) (xy -4.21203 7.688125)
    (xy -4.40088 7.879845) (xy -4.33778 7.967545) (xy -4.26108 8.047345) (xy -4.17208 8.118045) (xy -4.07218 8.178545)
    (xy -3.96276 8.227645) (xy -3.84518 8.264145) (xy -3.72084 8.286945) (xy -3.59109 8.294945) (xy -3.5907 8.295375))
   (layer F.Cu) (width 0))
  (fp_poly
   (pts (xy -1.10433 6.120635) (xy -1.10433 7.076375) (xy -2.24607 7.076375) (xy -2.24607 6.120635) (xy -2.50646 6.120635)
    (xy -2.50646 8.266755) (xy -2.24607 8.266755) (xy -2.24607 7.311015) (xy -1.10433 7.311015) (xy -1.10433 8.266755)
    (xy -0.84394 8.266755) (xy -0.84394 6.120635) (xy -1.10433 6.120635))
   (layer F.Cu) (width 0)))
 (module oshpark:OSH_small (layer F.Cu) (at 153.543 56.3245)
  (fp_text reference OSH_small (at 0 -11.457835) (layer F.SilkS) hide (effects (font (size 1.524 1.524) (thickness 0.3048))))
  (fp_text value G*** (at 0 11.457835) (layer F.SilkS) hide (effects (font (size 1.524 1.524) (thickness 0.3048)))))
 (gr_line (start 120.8405 40.64) (end 187.198 40.64) (layer Edge.Cuts) (width 0.12))
 (gr_line (start 118.0465 43.434) (end 118.11 64.3255) (layer Edge.Cuts) (width 0.12))
 (gr_line (start 187.198 67.056) (end 120.904 67.1195) (layer Edge.Cuts) (width 0.12))
 (gr_arc (start 120.904 64.3255) (end 118.11 64.3255) (angle -90) (layer Edge.Cuts) (width 0.12))
 (gr_arc (start 120.8405 43.434) (end 120.8405 40.64) (angle -90) (layer Edge.Cuts) (width 0.12))
 (gr_line (start 189.992 43.434) (end 189.992 64.262) (layer Edge.Cuts) (width 0.12))
 (gr_arc (start 187.198 43.434) (end 189.992 43.434) (angle -90) (layer Edge.Cuts) (width 0.12))
 (gr_arc (start 187.198 64.262) (end 187.198 67.056) (angle -90) (layer Edge.Cuts) (width 0.12))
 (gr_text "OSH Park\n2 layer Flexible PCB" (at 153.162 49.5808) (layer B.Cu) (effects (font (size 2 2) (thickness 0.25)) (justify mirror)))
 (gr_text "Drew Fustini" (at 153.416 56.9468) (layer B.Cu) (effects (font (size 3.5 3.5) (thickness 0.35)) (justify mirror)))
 (segment (start 125.6665 54.864) (end 125.6665 47.1805) (width 0.25) (layer B.Cu) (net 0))
 (segment (start 130.2245 42.6225) (end 153.4795 42.6225) (width 0.25) (layer B.Cu) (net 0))
 (segment (start 125.6665 47.1805) (end 130.2245 42.6225) (width 0.25) (layer B.Cu) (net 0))
 (via (at 153.4795 46.5455) (size 0.8) (drill 0.4) (layers F.Cu B.Cu) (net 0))
 (segment (start 153.4795 44.3725) (end 153.4795 46.5455) (width 0.25) (layer B.Cu) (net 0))
 (segment (start 153.4795 46.5455) (end 153.4795 53.848) (width 0.25) (layer F.Cu) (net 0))
 (via (at 154.813 54.8005) (size 0.8) (drill 0.4) (layers F.Cu B.Cu) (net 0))
 (segment (start 153.4795 55.598) (end 154.0155 55.598) (width 0.25) (layer F.Cu) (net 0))
 (segment (start 154.0155 55.598) (end 154.813 54.8005) (width 0.25) (layer F.Cu) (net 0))
 (segment (start 155.6385 53.975) (end 181.864 53.975) (width 0.25) (layer B.Cu) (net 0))
 (segment (start 154.813 54.8005) (end 155.6385 53.975) (width 0.25) (layer B.Cu) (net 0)))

